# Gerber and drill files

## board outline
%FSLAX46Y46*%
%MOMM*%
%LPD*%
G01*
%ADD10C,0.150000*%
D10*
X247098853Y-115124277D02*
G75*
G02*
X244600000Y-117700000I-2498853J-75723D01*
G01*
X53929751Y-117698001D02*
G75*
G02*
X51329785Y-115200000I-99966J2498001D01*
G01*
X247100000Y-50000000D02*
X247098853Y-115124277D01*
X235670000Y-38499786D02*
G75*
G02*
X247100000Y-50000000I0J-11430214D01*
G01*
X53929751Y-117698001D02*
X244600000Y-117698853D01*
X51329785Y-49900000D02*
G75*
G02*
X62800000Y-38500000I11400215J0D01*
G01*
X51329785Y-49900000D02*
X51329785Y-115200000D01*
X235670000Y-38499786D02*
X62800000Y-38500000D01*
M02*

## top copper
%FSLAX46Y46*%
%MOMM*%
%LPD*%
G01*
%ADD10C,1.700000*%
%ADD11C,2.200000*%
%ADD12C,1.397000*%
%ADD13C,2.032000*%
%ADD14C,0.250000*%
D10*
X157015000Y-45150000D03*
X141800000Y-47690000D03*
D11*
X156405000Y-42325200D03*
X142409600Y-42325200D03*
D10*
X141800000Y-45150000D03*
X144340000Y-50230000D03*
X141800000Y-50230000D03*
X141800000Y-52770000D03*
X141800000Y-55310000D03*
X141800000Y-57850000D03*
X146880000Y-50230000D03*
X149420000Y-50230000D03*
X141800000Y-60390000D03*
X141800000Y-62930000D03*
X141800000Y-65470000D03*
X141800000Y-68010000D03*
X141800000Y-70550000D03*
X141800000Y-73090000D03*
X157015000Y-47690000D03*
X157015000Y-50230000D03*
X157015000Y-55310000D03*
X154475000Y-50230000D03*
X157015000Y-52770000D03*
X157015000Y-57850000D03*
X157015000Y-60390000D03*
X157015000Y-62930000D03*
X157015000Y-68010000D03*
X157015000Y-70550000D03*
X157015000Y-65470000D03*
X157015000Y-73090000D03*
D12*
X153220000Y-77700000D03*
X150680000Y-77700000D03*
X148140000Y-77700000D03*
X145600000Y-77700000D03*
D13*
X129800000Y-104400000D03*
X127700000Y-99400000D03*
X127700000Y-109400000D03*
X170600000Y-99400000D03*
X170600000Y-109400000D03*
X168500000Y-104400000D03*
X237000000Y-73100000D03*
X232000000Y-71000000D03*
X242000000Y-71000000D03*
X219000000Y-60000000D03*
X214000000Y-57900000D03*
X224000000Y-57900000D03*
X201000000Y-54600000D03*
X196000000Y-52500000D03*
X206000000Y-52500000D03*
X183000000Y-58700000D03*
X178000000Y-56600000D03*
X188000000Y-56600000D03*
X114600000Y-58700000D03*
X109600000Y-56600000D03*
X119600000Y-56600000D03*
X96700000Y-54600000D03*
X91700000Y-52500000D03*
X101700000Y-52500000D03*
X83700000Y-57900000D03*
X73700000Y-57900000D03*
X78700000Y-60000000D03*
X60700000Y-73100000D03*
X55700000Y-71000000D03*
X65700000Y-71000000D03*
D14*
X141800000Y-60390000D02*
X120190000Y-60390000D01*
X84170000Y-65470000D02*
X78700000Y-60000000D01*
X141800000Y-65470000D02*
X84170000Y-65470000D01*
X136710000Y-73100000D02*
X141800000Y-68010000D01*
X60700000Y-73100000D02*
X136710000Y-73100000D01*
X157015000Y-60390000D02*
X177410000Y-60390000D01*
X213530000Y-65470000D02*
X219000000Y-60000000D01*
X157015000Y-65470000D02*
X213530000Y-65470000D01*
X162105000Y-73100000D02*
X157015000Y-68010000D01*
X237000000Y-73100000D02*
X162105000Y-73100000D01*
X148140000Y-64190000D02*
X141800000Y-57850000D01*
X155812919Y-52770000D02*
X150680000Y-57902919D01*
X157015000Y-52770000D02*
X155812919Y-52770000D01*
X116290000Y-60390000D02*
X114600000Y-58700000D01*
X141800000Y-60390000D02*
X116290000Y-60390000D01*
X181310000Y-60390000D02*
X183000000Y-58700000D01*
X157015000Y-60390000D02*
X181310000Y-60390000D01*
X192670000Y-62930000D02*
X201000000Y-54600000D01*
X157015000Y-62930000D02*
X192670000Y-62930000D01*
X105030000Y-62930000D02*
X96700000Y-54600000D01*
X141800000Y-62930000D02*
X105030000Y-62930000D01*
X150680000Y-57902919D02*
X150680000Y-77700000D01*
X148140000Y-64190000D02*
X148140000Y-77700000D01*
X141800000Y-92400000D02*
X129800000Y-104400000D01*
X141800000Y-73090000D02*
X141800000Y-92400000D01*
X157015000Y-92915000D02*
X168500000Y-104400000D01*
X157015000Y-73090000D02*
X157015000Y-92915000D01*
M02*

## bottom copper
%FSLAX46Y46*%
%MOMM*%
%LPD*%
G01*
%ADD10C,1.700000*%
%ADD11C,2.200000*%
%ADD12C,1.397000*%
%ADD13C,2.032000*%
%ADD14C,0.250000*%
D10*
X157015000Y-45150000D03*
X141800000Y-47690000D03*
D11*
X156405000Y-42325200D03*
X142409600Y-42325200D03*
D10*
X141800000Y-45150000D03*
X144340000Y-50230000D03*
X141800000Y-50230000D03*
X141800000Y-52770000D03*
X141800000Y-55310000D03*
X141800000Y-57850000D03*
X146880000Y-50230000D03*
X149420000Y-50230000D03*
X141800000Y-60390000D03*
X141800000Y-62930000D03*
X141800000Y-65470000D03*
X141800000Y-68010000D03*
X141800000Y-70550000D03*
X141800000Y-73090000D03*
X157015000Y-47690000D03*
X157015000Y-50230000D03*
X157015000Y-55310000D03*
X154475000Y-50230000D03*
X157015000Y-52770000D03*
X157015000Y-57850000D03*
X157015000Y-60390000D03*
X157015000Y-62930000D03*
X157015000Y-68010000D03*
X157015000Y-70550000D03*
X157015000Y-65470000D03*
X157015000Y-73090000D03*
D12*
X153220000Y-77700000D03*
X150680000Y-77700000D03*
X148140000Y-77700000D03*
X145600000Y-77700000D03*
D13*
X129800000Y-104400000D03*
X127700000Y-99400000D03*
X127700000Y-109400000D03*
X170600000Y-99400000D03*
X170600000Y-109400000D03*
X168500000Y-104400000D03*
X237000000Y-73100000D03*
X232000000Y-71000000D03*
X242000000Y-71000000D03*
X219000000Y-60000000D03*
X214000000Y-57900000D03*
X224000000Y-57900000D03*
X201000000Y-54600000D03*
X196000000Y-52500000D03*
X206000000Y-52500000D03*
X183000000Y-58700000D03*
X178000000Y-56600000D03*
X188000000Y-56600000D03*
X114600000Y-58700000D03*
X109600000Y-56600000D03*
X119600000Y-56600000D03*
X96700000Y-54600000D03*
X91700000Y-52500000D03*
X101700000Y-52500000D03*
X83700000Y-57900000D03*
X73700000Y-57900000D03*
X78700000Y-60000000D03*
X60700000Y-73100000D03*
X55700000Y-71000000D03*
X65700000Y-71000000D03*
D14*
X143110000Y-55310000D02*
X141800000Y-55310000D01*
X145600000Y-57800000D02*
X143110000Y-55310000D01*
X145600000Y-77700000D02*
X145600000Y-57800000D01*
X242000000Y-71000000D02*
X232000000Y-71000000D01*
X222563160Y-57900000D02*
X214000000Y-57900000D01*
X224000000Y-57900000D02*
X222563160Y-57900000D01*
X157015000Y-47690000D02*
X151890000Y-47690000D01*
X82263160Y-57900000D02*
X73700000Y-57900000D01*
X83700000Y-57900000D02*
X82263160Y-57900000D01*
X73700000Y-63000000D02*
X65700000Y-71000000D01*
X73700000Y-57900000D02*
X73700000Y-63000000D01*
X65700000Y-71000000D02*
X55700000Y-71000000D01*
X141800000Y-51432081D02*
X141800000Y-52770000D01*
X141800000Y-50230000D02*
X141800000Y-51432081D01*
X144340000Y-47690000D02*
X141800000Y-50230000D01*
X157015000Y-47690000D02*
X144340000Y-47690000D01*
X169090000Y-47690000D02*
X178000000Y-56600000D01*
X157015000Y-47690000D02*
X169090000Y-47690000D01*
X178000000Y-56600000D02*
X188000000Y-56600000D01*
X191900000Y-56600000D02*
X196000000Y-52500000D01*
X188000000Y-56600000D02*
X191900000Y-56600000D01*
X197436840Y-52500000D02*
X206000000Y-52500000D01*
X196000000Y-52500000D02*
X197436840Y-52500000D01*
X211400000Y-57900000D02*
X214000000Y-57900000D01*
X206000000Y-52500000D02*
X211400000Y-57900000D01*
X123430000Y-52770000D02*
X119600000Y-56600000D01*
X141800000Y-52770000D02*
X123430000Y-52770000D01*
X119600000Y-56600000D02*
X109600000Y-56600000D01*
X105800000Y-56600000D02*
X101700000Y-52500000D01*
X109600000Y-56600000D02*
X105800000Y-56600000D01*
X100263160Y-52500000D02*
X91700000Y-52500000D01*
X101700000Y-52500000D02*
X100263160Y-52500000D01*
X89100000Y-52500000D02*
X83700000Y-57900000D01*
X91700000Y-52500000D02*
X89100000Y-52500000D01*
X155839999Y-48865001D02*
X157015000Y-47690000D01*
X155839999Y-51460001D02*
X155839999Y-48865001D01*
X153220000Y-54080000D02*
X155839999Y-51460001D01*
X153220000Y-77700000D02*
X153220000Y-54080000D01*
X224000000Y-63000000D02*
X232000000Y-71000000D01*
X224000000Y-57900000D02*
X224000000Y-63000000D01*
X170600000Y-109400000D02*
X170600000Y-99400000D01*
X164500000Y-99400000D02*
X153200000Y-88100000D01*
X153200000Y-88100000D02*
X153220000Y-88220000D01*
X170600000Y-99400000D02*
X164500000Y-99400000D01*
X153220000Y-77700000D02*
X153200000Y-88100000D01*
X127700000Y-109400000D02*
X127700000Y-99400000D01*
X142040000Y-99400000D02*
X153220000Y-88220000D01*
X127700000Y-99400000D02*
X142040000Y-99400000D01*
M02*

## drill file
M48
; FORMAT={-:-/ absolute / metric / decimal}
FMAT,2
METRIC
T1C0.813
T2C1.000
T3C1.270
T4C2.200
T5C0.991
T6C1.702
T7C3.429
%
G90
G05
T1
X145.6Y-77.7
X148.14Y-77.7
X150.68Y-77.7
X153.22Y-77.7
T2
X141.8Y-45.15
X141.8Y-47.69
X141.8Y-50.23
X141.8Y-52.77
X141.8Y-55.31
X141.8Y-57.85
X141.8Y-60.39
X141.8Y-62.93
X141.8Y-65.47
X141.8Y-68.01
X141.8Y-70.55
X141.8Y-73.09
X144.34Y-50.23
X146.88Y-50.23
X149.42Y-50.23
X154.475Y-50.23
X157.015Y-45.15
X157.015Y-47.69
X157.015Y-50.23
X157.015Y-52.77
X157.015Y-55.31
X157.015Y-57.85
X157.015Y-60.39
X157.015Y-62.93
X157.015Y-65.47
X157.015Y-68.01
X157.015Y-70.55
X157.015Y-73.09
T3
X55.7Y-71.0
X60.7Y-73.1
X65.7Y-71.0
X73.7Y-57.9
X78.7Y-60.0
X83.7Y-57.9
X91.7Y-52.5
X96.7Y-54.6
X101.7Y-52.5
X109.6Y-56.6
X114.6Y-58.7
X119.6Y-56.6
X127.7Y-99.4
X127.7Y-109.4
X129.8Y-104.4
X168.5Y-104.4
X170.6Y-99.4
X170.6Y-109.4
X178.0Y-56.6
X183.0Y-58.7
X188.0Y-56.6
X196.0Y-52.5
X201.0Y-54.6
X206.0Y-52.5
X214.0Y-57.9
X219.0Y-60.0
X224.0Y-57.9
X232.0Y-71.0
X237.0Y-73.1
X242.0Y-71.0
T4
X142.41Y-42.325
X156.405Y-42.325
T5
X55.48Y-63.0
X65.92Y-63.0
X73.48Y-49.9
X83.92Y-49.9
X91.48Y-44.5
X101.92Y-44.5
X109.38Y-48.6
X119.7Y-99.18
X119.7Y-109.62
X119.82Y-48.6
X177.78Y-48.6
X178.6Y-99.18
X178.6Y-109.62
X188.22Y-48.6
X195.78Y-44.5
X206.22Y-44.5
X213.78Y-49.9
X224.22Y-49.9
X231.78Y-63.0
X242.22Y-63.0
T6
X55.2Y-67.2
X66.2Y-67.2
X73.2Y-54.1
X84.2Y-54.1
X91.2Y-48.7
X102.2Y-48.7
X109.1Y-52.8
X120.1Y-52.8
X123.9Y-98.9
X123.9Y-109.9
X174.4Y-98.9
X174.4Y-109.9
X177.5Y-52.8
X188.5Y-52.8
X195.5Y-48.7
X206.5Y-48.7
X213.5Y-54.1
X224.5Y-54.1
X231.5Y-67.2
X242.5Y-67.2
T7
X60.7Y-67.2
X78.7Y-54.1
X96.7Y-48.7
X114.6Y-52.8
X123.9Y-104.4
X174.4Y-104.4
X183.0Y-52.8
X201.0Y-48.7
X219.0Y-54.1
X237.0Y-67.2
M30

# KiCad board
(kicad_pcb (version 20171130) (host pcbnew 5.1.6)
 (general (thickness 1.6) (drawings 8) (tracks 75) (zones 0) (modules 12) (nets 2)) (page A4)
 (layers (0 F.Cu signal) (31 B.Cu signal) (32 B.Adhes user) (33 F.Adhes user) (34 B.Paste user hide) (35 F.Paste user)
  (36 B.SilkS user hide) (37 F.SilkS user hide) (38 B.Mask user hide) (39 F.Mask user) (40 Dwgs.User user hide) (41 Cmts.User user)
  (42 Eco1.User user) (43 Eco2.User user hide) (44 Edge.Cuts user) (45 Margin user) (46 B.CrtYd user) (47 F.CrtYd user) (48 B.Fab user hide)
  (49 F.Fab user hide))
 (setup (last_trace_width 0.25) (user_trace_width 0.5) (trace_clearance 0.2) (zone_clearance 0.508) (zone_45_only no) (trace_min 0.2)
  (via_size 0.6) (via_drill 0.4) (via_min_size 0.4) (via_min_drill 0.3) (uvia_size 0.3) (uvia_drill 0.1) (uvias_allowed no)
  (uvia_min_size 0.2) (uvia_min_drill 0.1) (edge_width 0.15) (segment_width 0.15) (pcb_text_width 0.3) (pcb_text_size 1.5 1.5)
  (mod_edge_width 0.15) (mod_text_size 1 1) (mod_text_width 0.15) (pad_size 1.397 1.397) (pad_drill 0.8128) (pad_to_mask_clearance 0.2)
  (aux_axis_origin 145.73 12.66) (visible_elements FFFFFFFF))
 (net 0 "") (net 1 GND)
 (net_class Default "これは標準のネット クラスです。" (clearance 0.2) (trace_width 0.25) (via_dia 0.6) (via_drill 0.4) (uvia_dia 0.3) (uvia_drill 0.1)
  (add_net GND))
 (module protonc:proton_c (layer F.Cu) (at 149.4 60.4)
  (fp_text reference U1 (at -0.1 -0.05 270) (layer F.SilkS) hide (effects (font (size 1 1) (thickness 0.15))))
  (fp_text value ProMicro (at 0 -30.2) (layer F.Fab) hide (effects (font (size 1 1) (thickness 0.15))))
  (pad 5V thru_hole circle (at 7.615 -15.25) (size 1.7 1.7) (drill 1) (layers *.Cu *.Mask))
  (pad A10 thru_hole circle (at -7.6 -12.71) (size 1.7 1.7) (drill 1) (layers *.Cu *.Mask))
  (pad SCRE thru_hole circle (at 7.005 -18.0748) (size 2.2 2.2) (drill 2.2) (layers *.Cu *.Mask))
  (pad SCRE thru_hole circle (at -6.9904 -18.0748) (size 2.2 2.2) (drill 2.2) (layers *.Cu *.Mask))
  (pad A9 thru_hole circle (at -7.6 -15.25) (size 1.7 1.7) (drill 1) (layers *.Cu *.Mask))
  (pad D+ thru_hole circle (at -5.06 -10.17) (size 1.7 1.7) (drill 1) (layers *.Cu *.Mask))
  (pad GND thru_hole circle (at -7.6 -10.17) (size 1.7 1.7) (drill 1) (layers *.Cu *.Mask) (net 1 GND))
  (pad GND thru_hole circle (at -7.6 -7.63) (size 1.7 1.7) (drill 1) (layers *.Cu *.Mask) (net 1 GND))
  (pad B7 thru_hole circle (at -7.6 -5.09) (size 1.7 1.7) (drill 1) (layers *.Cu *.Mask))
  (pad B6 thru_hole circle (at -7.6 -2.55) (size 1.7 1.7) (drill 1) (layers *.Cu *.Mask))
  (pad D- thru_hole circle (at -2.52 -10.17) (size 1.7 1.7) (drill 1) (layers *.Cu *.Mask))
  (pad CHRG thru_hole circle (at 0.02 -10.17) (size 1.7 1.7) (drill 1) (layers *.Cu *.Mask))
  (pad B5 thru_hole circle (at -7.6 -0.01) (size 1.7 1.7) (drill 1) (layers *.Cu *.Mask))
  (pad B4 thru_hole circle (at -7.6 2.53) (size 1.7 1.7) (drill 1) (layers *.Cu *.Mask))
  (pad B3 thru_hole circle (at -7.6 5.07) (size 1.7 1.7) (drill 1) (layers *.Cu *.Mask))
  (pad B2 thru_hole circle (at -7.6 7.61) (size 1.7 1.7) (drill 1) (layers *.Cu *.Mask))
  (pad B1 thru_hole circle (at -7.6 10.15) (size 1.7 1.7) (drill 1) (layers *.Cu *.Mask))
  (pad B0 thru_hole circle (at -7.6 12.69) (size 1.7 1.7) (drill 1) (layers *.Cu *.Mask))
  (pad GND thru_hole circle (at 7.615 -12.71) (size 1.7 1.7) (drill 1) (layers *.Cu *.Mask) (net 1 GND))
  (pad DFU thru_hole circle (at 7.615 -10.17) (size 1.7 1.7) (drill 1) (layers *.Cu *.Mask))
  (pad A2 thru_hole circle (at 7.615 -5.09) (size 1.7 1.7) (drill 1) (layers *.Cu *.Mask))
  (pad A3|5v thru_hole circle (at 5.075 -10.17) (size 1.7 1.7) (drill 1) (layers *.Cu *.Mask))
  (pad 3.3V thru_hole circle (at 7.615 -7.63) (size 1.7 1.7) (drill 1) (layers *.Cu *.Mask))
  (pad A1 thru_hole circle (at 7.615 -2.55) (size 1.7 1.7) (drill 1) (layers *.Cu *.Mask))
  (pad A0 thru_hole circle (at 7.615 -0.01) (size 1.7 1.7) (drill 1) (layers *.Cu *.Mask))
  (pad B8 thru_hole circle (at 7.615 2.53) (size 1.7 1.7) (drill 1) (layers *.Cu *.Mask))
  (pad B14 thru_hole circle (at 7.615 7.61) (size 1.7 1.7) (drill 1) (layers *.Cu *.Mask))
  (pad B15 thru_hole circle (at 7.615 10.15) (size 1.7 1.7) (drill 1) (layers *.Cu *.Mask))
  (pad B13 thru_hole circle (at 7.615 5.07) (size 1.7 1.7) (drill 1) (layers *.Cu *.Mask))
  (pad B9 thru_hole circle (at 7.615 12.69) (size 1.7 1.7) (drill 1) (layers *.Cu *.Mask)))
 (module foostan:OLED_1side (layer F.Cu) (at 145.6 77.7)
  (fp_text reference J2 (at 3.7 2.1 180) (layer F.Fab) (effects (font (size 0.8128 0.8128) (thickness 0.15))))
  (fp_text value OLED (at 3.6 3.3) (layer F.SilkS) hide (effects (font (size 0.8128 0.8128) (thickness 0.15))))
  (pad 4 thru_hole circle (at 7.62 0) (size 1.397 1.397) (drill 0.8128) (layers *.Cu F.SilkS B.Mask) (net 1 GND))
  (pad 3 thru_hole circle (at 5.08 0) (size 1.397 1.397) (drill 0.8128) (layers *.Cu F.SilkS B.Mask))
  (pad 2 thru_hole circle (at 2.54 0) (size 1.397 1.397) (drill 0.8128) (layers *.Cu F.SilkS B.Mask))
  (pad 1 thru_hole circle (at 0 0) (size 1.397 1.397) (drill 0.8128) (layers *.Cu F.SilkS B.Mask)))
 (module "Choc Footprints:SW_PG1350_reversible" (layer B.Cu) (at 123.9 104.4 270)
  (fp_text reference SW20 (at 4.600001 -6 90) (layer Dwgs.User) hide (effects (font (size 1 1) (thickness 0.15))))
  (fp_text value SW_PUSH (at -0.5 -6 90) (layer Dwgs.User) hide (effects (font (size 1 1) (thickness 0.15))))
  (pad "" np_thru_hole circle (at -5.5 0 270) (size 1.7018 1.7018) (drill 1.7018) (layers *.Cu *.Mask))
  (pad "" np_thru_hole circle (at 5.5 0 270) (size 1.7018 1.7018) (drill 1.7018) (layers *.Cu *.Mask))
  (pad "" np_thru_hole circle (at 5.22 4.2 270) (size 0.9906 0.9906) (drill 0.9906) (layers *.Cu *.Mask))
  (pad 1 thru_hole circle (at 0 -5.9 270) (size 2.032 2.032) (drill 1.27) (layers *.Cu *.Mask))
  (pad 2 thru_hole circle (at -5 -3.8 270) (size 2.032 2.032) (drill 1.27) (layers *.Cu *.Mask) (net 1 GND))
  (pad "" np_thru_hole circle (at 0 0 270) (size 3.429 3.429) (drill 3.429) (layers *.Cu *.Mask))
  (pad 2 thru_hole circle (at 5 -3.8 270) (size 2.032 2.032) (drill 1.27) (layers *.Cu *.Mask) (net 1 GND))
  (pad "" np_thru_hole circle (at -5.22 4.2 270) (size 0.9906 0.9906) (drill 0.9906) (layers *.Cu *.Mask)))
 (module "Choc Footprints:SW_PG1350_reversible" (layer B.Cu) (at 174.4 104.4 90)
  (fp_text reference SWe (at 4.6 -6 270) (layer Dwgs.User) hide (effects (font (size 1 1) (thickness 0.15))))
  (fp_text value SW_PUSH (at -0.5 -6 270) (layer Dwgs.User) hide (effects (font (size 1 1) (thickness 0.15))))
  (pad "" np_thru_hole circle (at -5.22 4.2 90) (size 0.9906 0.9906) (drill 0.9906) (layers *.Cu *.Mask))
  (pad 2 thru_hole circle (at 5 -3.8 90) (size 2.032 2.032) (drill 1.27) (layers *.Cu *.Mask) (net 1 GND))
  (pad "" np_thru_hole circle (at 0 0 90) (size 3.429 3.429) (drill 3.429) (layers *.Cu *.Mask))
  (pad 2 thru_hole circle (at -5 -3.8 90) (size 2.032 2.032) (drill 1.27) (layers *.Cu *.Mask) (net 1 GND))
  (pad 1 thru_hole circle (at 0 -5.9 90) (size 2.032 2.032) (drill 1.27) (layers *.Cu *.Mask))
  (pad "" np_thru_hole circle (at 5.22 4.2 90) (size 0.9906 0.9906) (drill 0.9906) (layers *.Cu *.Mask))
  (pad "" np_thru_hole circle (at 5.5 0 90) (size 1.7018 1.7018) (drill 1.7018) (layers *.Cu *.Mask))
  (pad "" np_thru_hole circle (at -5.5 0 90) (size 1.7018 1.7018) (drill 1.7018) (layers *.Cu *.Mask)))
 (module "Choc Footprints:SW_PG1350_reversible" (layer F.Cu) (at 237 67.2)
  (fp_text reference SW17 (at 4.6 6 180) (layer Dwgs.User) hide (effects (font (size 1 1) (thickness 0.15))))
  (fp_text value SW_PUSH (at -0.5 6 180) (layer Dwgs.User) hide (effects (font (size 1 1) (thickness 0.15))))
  (pad "" np_thru_hole circle (at -5.5 0) (size 1.7018 1.7018) (drill 1.7018) (layers *.Cu *.Mask))
  (pad "" np_thru_hole circle (at 5.5 0) (size 1.7018 1.7018) (drill 1.7018) (layers *.Cu *.Mask))
  (pad "" np_thru_hole circle (at 5.22 -4.2) (size 0.9906 0.9906) (drill 0.9906) (layers *.Cu *.Mask))
  (pad 1 thru_hole circle (at 0 5.9) (size 2.032 2.032) (drill 1.27) (layers *.Cu *.Mask))
  (pad 2 thru_hole circle (at -5 3.8) (size 2.032 2.032) (drill 1.27) (layers *.Cu *.Mask) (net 1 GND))
  (pad "" np_thru_hole circle (at 0 0) (size 3.429 3.429) (drill 3.429) (layers *.Cu *.Mask))
  (pad 2 thru_hole circle (at 5 3.8) (size 2.032 2.032) (drill 1.27) (layers *.Cu *.Mask) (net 1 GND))
  (pad "" np_thru_hole circle (at -5.22 -4.2) (size 0.9906 0.9906) (drill 0.9906) (layers *.Cu *.Mask)))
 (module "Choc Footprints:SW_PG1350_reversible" (layer F.Cu) (at 219 54.1)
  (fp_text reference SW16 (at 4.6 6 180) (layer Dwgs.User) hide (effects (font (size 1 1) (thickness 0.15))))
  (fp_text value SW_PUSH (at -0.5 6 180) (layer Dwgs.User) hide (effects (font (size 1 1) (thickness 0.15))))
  (pad "" np_thru_hole circle (at -5.5 0) (size 1.7018 1.7018) (drill 1.7018) (layers *.Cu *.Mask))
  (pad "" np_thru_hole circle (at 5.5 0) (size 1.7018 1.7018) (drill 1.7018) (layers *.Cu *.Mask))
  (pad "" np_thru_hole circle (at 5.22 -4.2) (size 0.9906 0.9906) (drill 0.9906) (layers *.Cu *.Mask))
  (pad 1 thru_hole circle (at 0 5.9) (size 2.032 2.032) (drill 1.27) (layers *.Cu *.Mask))
  (pad 2 thru_hole circle (at -5 3.8) (size 2.032 2.032) (drill 1.27) (layers *.Cu *.Mask) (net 1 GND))
  (pad "" np_thru_hole circle (at 0 0) (size 3.429 3.429) (drill 3.429) (layers *.Cu *.Mask))
  (pad 2 thru_hole circle (at 5 3.8) (size 2.032 2.032) (drill 1.27) (layers *.Cu *.Mask) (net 1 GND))
  (pad "" np_thru_hole circle (at -5.22 -4.2) (size 0.9906 0.9906) (drill 0.9906) (layers *.Cu *.Mask)))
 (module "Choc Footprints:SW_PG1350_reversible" (layer F.Cu) (at 201 48.7)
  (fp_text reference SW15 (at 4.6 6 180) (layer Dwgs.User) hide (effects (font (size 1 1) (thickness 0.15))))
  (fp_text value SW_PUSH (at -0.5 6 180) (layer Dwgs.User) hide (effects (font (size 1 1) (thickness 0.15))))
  (pad "" np_thru_hole circle (at -5.5 0) (size 1.7018 1.7018) (drill 1.7018) (layers *.Cu *.Mask))
  (pad "" np_thru_hole circle (at 5.5 0) (size 1.7018 1.7018) (drill 1.7018) (layers *.Cu *.Mask))
  (pad "" np_thru_hole circle (at 5.22 -4.2) (size 0.9906 0.9906) (drill 0.9906) (layers *.Cu *.Mask))
  (pad 1 thru_hole circle (at 0 5.9) (size 2.032 2.032) (drill 1.27) (layers *.Cu *.Mask))
  (pad 2 thru_hole circle (at -5 3.8) (size 2.032 2.032) (drill 1.27) (layers *.Cu *.Mask) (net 1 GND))
  (pad "" np_thru_hole circle (at 0 0) (size 3.429 3.429) (drill 3.429) (layers *.Cu *.Mask))
  (pad 2 thru_hole circle (at 5 3.8) (size 2.032 2.032) (drill 1.27) (layers *.Cu *.Mask) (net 1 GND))
  (pad "" np_thru_hole circle (at -5.22 -4.2) (size 0.9906 0.9906) (drill 0.9906) (layers *.Cu *.Mask)))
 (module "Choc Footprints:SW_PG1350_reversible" (layer F.Cu) (at 183 52.8)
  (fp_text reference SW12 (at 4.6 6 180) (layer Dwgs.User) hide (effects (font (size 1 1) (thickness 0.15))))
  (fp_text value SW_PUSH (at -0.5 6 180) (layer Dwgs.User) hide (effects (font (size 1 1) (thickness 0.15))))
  (pad "" np_thru_hole circle (at -5.5 0) (size 1.7018 1.7018) (drill 1.7018) (layers *.Cu *.Mask))
  (pad "" np_thru_hole circle (at 5.5 0) (size 1.7018 1.7018) (drill 1.7018) (layers *.Cu *.Mask))
  (pad "" np_thru_hole circle (at 5.22 -4.2) (size 0.9906 0.9906) (drill 0.9906) (layers *.Cu *.Mask))
  (pad 1 thru_hole circle (at 0 5.9) (size 2.032 2.032) (drill 1.27) (layers *.Cu *.Mask))
  (pad 2 thru_hole circle (at -5 3.8) (size 2.032 2.032) (drill 1.27) (layers *.Cu *.Mask) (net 1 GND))
  (pad "" np_thru_hole circle (at 0 0) (size 3.429 3.429) (drill 3.429) (layers *.Cu *.Mask))
  (pad 2 thru_hole circle (at 5 3.8) (size 2.032 2.032) (drill 1.27) (layers *.Cu *.Mask) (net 1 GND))
  (pad "" np_thru_hole circle (at -5.22 -4.2) (size 0.9906 0.9906) (drill 0.9906) (layers *.Cu *.Mask)))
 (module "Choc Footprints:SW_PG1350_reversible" (layer F.Cu) (at 114.6 52.8)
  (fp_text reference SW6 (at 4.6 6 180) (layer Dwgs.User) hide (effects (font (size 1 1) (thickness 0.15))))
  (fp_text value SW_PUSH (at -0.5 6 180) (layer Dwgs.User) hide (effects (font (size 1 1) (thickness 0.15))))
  (pad "" np_thru_hole circle (at -5.5 0) (size 1.7018 1.7018) (drill 1.7018) (layers *.Cu *.Mask))
  (pad "" np_thru_hole circle (at 5.5 0) (size 1.7018 1.7018) (drill 1.7018) (layers *.Cu *.Mask))
  (pad "" np_thru_hole circle (at 5.22 -4.2) (size 0.9906 0.9906) (drill 0.9906) (layers *.Cu *.Mask))
  (pad 1 thru_hole circle (at 0 5.9) (size 2.032 2.032) (drill 1.27) (layers *.Cu *.Mask))
  (pad 2 thru_hole circle (at -5 3.8) (size 2.032 2.032) (drill 1.27) (layers *.Cu *.Mask) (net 1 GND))
  (pad "" np_thru_hole circle (at 0 0) (size 3.429 3.429) (drill 3.429) (layers *.Cu *.Mask))
  (pad 2 thru_hole circle (at 5 3.8) (size 2.032 2.032) (drill 1.27) (layers *.Cu *.Mask) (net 1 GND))
  (pad "" np_thru_hole circle (at -5.22 -4.2) (size 0.9906 0.9906) (drill 0.9906) (layers *.Cu *.Mask)))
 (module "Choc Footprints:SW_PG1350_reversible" (layer F.Cu) (at 96.7 48.7)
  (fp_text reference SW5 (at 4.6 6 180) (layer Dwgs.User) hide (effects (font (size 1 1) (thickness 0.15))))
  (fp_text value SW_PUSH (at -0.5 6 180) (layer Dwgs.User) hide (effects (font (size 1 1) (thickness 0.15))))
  (pad "" np_thru_hole circle (at -5.5 0) (size 1.7018 1.7018) (drill 1.7018) (layers *.Cu *.Mask))
  (pad "" np_thru_hole circle (at 5.5 0) (size 1.7018 1.7018) (drill 1.7018) (layers *.Cu *.Mask))
  (pad "" np_thru_hole circle (at 5.22 -4.2) (size 0.9906 0.9906) (drill 0.9906) (layers *.Cu *.Mask))
  (pad 1 thru_hole circle (at 0 5.9) (size 2.032 2.032) (drill 1.27) (layers *.Cu *.Mask))
  (pad 2 thru_hole circle (at -5 3.8) (size 2.032 2.032) (drill 1.27) (layers *.Cu *.Mask) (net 1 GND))
  (pad "" np_thru_hole circle (at 0 0) (size 3.429 3.429) (drill 3.429) (layers *.Cu *.Mask))
  (pad 2 thru_hole circle (at 5 3.8) (size 2.032 2.032) (drill 1.27) (layers *.Cu *.Mask) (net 1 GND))
  (pad "" np_thru_hole circle (at -5.22 -4.2) (size 0.9906 0.9906) (drill 0.9906) (layers *.Cu *.Mask)))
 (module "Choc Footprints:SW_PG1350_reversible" (layer F.Cu) (at 78.7 54.1)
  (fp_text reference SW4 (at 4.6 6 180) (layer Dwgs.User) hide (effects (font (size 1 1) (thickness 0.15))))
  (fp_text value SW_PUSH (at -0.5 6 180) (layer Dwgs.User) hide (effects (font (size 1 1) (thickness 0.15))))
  (pad "" np_thru_hole circle (at -5.22 -4.2) (size 0.9906 0.9906) (drill 0.9906) (layers *.Cu *.Mask))
  (pad 2 thru_hole circle (at 5 3.8) (size 2.032 2.032) (drill 1.27) (layers *.Cu *.Mask) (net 1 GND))
  (pad "" np_thru_hole circle (at 0 0) (size 3.429 3.429) (drill 3.429) (layers *.Cu *.Mask))
  (pad 2 thru_hole circle (at -5 3.8) (size 2.032 2.032) (drill 1.27) (layers *.Cu *.Mask) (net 1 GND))
  (pad 1 thru_hole circle (at 0 5.9) (size 2.032 2.032) (drill 1.27) (layers *.Cu *.Mask))
  (pad "" np_thru_hole circle (at 5.22 -4.2) (size 0.9906 0.9906) (drill 0.9906) (layers *.Cu *.Mask))
  (pad "" np_thru_hole circle (at 5.5 0) (size 1.7018 1.7018) (drill 1.7018) (layers *.Cu *.Mask))
  (pad "" np_thru_hole circle (at -5.5 0) (size 1.7018 1.7018) (drill 1.7018) (layers *.Cu *.Mask)))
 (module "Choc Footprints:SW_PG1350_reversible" (layer F.Cu) (at 60.7 67.2)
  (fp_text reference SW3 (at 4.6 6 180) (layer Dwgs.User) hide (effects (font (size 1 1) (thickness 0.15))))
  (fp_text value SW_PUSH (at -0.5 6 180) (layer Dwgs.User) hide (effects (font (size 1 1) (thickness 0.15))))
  (pad "" np_thru_hole circle (at -5.5 0) (size 1.7018 1.7018) (drill 1.7018) (layers *.Cu *.Mask))
  (pad "" np_thru_hole circle (at 5.5 0) (size 1.7018 1.7018) (drill 1.7018) (layers *.Cu *.Mask))
  (pad "" np_thru_hole circle (at 5.22 -4.2) (size 0.9906 0.9906) (drill 0.9906) (layers *.Cu *.Mask))
  (pad 1 thru_hole circle (at 0 5.9) (size 2.032 2.032) (drill 1.27) (layers *.Cu *.Mask))
  (pad 2 thru_hole circle (at -5 3.8) (size 2.032 2.032) (drill 1.27) (layers *.Cu *.Mask) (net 1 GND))
  (pad "" np_thru_hole circle (at 0 0) (size 3.429 3.429) (drill 3.429) (layers *.Cu *.Mask))
  (pad 2 thru_hole circle (at 5 3.8) (size 2.032 2.032) (drill 1.27) (layers *.Cu *.Mask) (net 1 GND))
  (pad "" np_thru_hole circle (at -5.22 -4.2) (size 0.9906 0.9906) (drill 0.9906) (layers *.Cu *.Mask)))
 (gr_arc (start 244.6 115.2) (end 244.6 117.7) (angle -91.73570459) (layer Edge.Cuts) (width 0.15))
 (gr_arc (start 53.829785 115.2) (end 51.329785 115.2) (angle -92.29166034) (layer Edge.Cuts) (width 0.15))
 (gr_line (start 247.1 50) (end 247.098853 115.124277) (angle 90) (layer Edge.Cuts) (width 0.15))
 (gr_arc (start 235.67 49.93) (end 247.1 50) (angle -90.3508884) (layer Edge.Cuts) (width 0.15))
 (gr_line (start 53.929751 117.698001) (end 244.6 117.698853) (angle 90) (layer Edge.Cuts) (width 0.15))
 (gr_arc (start 62.73 49.9) (end 62.8 38.5) (angle -90.35181177) (layer Edge.Cuts) (width 0.15))
 (gr_line (start 51.329785 49.9) (end 51.329785 115.2) (angle 90) (layer Edge.Cuts) (width 0.15))
 (gr_line (start 235.67 38.499786) (end 62.8 38.5) (angle 90) (layer Edge.Cuts) (width 0.15))
 (segment (start 141.8 60.39) (end 120.19 60.39) (width 0.25) (layer F.Cu) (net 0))
 (segment (start 84.17 65.47) (end 78.7 60) (width 0.25) (layer F.Cu) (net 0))
 (segment (start 141.8 65.47) (end 84.17 65.47) (width 0.25) (layer F.Cu) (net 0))
 (segment (start 136.71 73.1) (end 141.8 68.01) (width 0.25) (layer F.Cu) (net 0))
 (segment (start 60.7 73.1) (end 136.71 73.1) (width 0.25) (layer F.Cu) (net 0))
 (segment (start 157.015 60.39) (end 177.41 60.39) (width 0.25) (layer F.Cu) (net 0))
 (segment (start 213.53 65.47) (end 219 60) (width 0.25) (layer F.Cu) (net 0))
 (segment (start 157.015 65.47) (end 213.53 65.47) (width 0.25) (layer F.Cu) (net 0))
 (segment (start 162.105 73.1) (end 157.015 68.01) (width 0.25) (layer F.Cu) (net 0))
 (segment (start 237 73.1) (end 162.105 73.1) (width 0.25) (layer F.Cu) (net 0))
 (segment (start 148.14 64.19) (end 141.8 57.85) (width 0.25) (layer F.Cu) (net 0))
 (segment (start 155.812919 52.77) (end 150.68 57.902919) (width 0.25) (layer F.Cu) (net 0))
 (segment (start 157.015 52.77) (end 155.812919 52.77) (width 0.25) (layer F.Cu) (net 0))
 (segment (start 116.29 60.39) (end 114.6 58.7) (width 0.25) (layer F.Cu) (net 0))
 (segment (start 141.8 60.39) (end 116.29 60.39) (width 0.25) (layer F.Cu) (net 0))
 (segment (start 181.31 60.39) (end 183 58.7) (width 0.25) (layer F.Cu) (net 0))
 (segment (start 157.015 60.39) (end 181.31 60.39) (width 0.25) (layer F.Cu) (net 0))
 (segment (start 192.67 62.93) (end 201 54.6) (width 0.25) (layer F.Cu) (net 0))
 (segment (start 157.015 62.93) (end 192.67 62.93) (width 0.25) (layer F.Cu) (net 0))
 (segment (start 105.03 62.93) (end 96.7 54.6) (width 0.25) (layer F.Cu) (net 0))
 (segment (start 141.8 62.93) (end 105.03 62.93) (width 0.25) (layer F.Cu) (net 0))
 (segment (start 143.11 55.31) (end 141.8 55.31) (width 0.25) (layer B.Cu) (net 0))
 (segment (start 145.6 57.8) (end 143.11 55.31) (width 0.25) (layer B.Cu) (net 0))
 (segment (start 145.6 77.7) (end 145.6 57.8) (width 0.25) (layer B.Cu) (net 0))
 (segment (start 150.68 57.902919) (end 150.68 77.7) (width 0.25) (layer F.Cu) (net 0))
 (segment (start 148.14 64.19) (end 148.14 77.7) (width 0.25) (layer F.Cu) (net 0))
 (segment (start 141.8 92.4) (end 129.8 104.4) (width 0.25) (layer F.Cu) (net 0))
 (segment (start 141.8 73.09) (end 141.8 92.4) (width 0.25) (layer F.Cu) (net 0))
 (segment (start 157.015 92.915) (end 168.5 104.4) (width 0.25) (layer F.Cu) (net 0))
 (segment (start 157.015 73.09) (end 157.015 92.915) (width 0.25) (layer F.Cu) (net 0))
 (segment (start 242 71) (end 232 71) (width 0.25) (layer B.Cu) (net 1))
 (segment (start 222.56316 57.9) (end 214 57.9) (width 0.25) (layer B.Cu) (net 1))
 (segment (start 224 57.9) (end 222.56316 57.9) (width 0.25) (layer B.Cu) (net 1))
 (segment (start 157.015 47.69) (end 151.89 47.69) (width 0.25) (layer B.Cu) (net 1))
 (segment (start 82.26316 57.9) (end 73.7 57.9) (width 0.25) (layer B.Cu) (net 1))
 (segment (start 83.7 57.9) (end 82.26316 57.9) (width 0.25) (layer B.Cu) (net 1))
 (segment (start 73.7 63) (end 65.7 71) (width 0.25) (layer B.Cu) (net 1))
 (segment (start 73.7 57.9) (end 73.7 63) (width 0.25) (layer B.Cu) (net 1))
 (segment (start 65.7 71) (end 55.7 71) (width 0.25) (layer B.Cu) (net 1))
 (segment (start 141.8 51.432081) (end 141.8 52.77) (width 0.25) (layer B.Cu) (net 1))
 (segment (start 141.8 50.23) (end 141.8 51.432081) (width 0.25) (layer B.Cu) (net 1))
 (segment (start 144.34 47.69) (end 141.8 50.23) (width 0.25) (layer B.Cu) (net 1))
 (segment (start 157.015 47.69) (end 144.34 47.69) (width 0.25) (layer B.Cu) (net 1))
 (segment (start 169.09 47.69) (end 178 56.6) (width 0.25) (layer B.Cu) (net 1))
 (segment (start 157.015 47.69) (end 169.09 47.69) (width 0.25) (layer B.Cu) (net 1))
 (segment (start 178 56.6) (end 188 56.6) (width 0.25) (layer B.Cu) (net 1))
 (segment (start 191.9 56.6) (end 196 52.5) (width 0.25) (layer B.Cu) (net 1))
 (segment (start 188 56.6) (end 191.9 56.6) (width 0.25) (layer B.Cu) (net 1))
 (segment (start 197.43684 52.5) (end 206 52.5) (width 0.25) (layer B.Cu) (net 1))
 (segment (start 196 52.5) (end 197.43684 52.5) (width 0.25) (layer B.Cu) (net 1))
 (segment (start 211.4 57.9) (end 214 57.9) (width 0.25) (layer B.Cu) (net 1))
 (segment (start 206 52.5) (end 211.4 57.9) (width 0.25) (layer B.Cu) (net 1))
 (segment (start 123.43 52.77) (end 119.6 56.6) (width 0.25) (layer B.Cu) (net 1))
 (segment (start 141.8 52.77) (end 123.43 52.77) (width 0.25) (layer B.Cu) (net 1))
 (segment (start 119.6 56.6) (end 109.6 56.6) (width 0.25) (layer B.Cu) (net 1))
 (segment (start 105.8 56.6) (end 101.7 52.5) (width 0.25) (layer B.Cu) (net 1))
 (segment (start 109.6 56.6) (end 105.8 56.6) (width 0.25) (layer B.Cu) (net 1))
 (segment (start 100.26316 52.5) (end 91.7 52.5) (width 0.25) (layer B.Cu) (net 1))
 (segment (start 101.7 52.5) (end 100.26316 52.5) (width 0.25) (layer B.Cu) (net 1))
 (segment (start 89.1 52.5) (end 83.7 57.9) (width 0.25) (layer B.Cu) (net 1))
 (segment (start 91.7 52.5) (end 89.1 52.5) (width 0.25) (layer B.Cu) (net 1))
 (segment (start 155.839999 48.865001) (end 157.015 47.69) (width 0.25) (layer B.Cu) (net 1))
 (segment (start 155.839999 51.460001) (end 155.839999 48.865001) (width 0.25) (layer B.Cu) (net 1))
 (segment (start 153.22 54.08) (end 155.839999 51.460001) (width 0.25) (layer B.Cu) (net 1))
 (segment (start 153.22 77.7) (end 153.22 54.08) (width 0.25) (layer B.Cu) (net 1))
 (segment (start 224 63) (end 232 71) (width 0.25) (layer B.Cu) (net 1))
 (segment (start 224 57.9) (end 224 63) (width 0.25) (layer B.Cu) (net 1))
 (segment (start 170.6 109.4) (end 170.6 99.4) (width 0.25) (layer B.Cu) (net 1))
 (segment (start 164.5 99.4) (end 153.2 88.1) (width 0.25) (layer B.Cu) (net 1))
 (segment (start 153.2 88.1) (end 153.22 88.22) (width 0.25) (layer B.Cu) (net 1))
 (segment (start 170.6 99.4) (end 164.5 99.4) (width 0.25) (layer B.Cu) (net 1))
 (segment (start 153.22 77.7) (end 153.2 88.1) (width 0.25) (layer B.Cu) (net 1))
 (segment (start 127.7 109.4) (end 127.7 99.4) (width 0.25) (layer B.Cu) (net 1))
 (segment (start 142.04 99.4) (end 153.22 88.22) (width 0.25) (layer B.Cu) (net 1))
 (segment (start 127.7 99.4) (end 142.04 99.4) (width 0.25) (layer B.Cu) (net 1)))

